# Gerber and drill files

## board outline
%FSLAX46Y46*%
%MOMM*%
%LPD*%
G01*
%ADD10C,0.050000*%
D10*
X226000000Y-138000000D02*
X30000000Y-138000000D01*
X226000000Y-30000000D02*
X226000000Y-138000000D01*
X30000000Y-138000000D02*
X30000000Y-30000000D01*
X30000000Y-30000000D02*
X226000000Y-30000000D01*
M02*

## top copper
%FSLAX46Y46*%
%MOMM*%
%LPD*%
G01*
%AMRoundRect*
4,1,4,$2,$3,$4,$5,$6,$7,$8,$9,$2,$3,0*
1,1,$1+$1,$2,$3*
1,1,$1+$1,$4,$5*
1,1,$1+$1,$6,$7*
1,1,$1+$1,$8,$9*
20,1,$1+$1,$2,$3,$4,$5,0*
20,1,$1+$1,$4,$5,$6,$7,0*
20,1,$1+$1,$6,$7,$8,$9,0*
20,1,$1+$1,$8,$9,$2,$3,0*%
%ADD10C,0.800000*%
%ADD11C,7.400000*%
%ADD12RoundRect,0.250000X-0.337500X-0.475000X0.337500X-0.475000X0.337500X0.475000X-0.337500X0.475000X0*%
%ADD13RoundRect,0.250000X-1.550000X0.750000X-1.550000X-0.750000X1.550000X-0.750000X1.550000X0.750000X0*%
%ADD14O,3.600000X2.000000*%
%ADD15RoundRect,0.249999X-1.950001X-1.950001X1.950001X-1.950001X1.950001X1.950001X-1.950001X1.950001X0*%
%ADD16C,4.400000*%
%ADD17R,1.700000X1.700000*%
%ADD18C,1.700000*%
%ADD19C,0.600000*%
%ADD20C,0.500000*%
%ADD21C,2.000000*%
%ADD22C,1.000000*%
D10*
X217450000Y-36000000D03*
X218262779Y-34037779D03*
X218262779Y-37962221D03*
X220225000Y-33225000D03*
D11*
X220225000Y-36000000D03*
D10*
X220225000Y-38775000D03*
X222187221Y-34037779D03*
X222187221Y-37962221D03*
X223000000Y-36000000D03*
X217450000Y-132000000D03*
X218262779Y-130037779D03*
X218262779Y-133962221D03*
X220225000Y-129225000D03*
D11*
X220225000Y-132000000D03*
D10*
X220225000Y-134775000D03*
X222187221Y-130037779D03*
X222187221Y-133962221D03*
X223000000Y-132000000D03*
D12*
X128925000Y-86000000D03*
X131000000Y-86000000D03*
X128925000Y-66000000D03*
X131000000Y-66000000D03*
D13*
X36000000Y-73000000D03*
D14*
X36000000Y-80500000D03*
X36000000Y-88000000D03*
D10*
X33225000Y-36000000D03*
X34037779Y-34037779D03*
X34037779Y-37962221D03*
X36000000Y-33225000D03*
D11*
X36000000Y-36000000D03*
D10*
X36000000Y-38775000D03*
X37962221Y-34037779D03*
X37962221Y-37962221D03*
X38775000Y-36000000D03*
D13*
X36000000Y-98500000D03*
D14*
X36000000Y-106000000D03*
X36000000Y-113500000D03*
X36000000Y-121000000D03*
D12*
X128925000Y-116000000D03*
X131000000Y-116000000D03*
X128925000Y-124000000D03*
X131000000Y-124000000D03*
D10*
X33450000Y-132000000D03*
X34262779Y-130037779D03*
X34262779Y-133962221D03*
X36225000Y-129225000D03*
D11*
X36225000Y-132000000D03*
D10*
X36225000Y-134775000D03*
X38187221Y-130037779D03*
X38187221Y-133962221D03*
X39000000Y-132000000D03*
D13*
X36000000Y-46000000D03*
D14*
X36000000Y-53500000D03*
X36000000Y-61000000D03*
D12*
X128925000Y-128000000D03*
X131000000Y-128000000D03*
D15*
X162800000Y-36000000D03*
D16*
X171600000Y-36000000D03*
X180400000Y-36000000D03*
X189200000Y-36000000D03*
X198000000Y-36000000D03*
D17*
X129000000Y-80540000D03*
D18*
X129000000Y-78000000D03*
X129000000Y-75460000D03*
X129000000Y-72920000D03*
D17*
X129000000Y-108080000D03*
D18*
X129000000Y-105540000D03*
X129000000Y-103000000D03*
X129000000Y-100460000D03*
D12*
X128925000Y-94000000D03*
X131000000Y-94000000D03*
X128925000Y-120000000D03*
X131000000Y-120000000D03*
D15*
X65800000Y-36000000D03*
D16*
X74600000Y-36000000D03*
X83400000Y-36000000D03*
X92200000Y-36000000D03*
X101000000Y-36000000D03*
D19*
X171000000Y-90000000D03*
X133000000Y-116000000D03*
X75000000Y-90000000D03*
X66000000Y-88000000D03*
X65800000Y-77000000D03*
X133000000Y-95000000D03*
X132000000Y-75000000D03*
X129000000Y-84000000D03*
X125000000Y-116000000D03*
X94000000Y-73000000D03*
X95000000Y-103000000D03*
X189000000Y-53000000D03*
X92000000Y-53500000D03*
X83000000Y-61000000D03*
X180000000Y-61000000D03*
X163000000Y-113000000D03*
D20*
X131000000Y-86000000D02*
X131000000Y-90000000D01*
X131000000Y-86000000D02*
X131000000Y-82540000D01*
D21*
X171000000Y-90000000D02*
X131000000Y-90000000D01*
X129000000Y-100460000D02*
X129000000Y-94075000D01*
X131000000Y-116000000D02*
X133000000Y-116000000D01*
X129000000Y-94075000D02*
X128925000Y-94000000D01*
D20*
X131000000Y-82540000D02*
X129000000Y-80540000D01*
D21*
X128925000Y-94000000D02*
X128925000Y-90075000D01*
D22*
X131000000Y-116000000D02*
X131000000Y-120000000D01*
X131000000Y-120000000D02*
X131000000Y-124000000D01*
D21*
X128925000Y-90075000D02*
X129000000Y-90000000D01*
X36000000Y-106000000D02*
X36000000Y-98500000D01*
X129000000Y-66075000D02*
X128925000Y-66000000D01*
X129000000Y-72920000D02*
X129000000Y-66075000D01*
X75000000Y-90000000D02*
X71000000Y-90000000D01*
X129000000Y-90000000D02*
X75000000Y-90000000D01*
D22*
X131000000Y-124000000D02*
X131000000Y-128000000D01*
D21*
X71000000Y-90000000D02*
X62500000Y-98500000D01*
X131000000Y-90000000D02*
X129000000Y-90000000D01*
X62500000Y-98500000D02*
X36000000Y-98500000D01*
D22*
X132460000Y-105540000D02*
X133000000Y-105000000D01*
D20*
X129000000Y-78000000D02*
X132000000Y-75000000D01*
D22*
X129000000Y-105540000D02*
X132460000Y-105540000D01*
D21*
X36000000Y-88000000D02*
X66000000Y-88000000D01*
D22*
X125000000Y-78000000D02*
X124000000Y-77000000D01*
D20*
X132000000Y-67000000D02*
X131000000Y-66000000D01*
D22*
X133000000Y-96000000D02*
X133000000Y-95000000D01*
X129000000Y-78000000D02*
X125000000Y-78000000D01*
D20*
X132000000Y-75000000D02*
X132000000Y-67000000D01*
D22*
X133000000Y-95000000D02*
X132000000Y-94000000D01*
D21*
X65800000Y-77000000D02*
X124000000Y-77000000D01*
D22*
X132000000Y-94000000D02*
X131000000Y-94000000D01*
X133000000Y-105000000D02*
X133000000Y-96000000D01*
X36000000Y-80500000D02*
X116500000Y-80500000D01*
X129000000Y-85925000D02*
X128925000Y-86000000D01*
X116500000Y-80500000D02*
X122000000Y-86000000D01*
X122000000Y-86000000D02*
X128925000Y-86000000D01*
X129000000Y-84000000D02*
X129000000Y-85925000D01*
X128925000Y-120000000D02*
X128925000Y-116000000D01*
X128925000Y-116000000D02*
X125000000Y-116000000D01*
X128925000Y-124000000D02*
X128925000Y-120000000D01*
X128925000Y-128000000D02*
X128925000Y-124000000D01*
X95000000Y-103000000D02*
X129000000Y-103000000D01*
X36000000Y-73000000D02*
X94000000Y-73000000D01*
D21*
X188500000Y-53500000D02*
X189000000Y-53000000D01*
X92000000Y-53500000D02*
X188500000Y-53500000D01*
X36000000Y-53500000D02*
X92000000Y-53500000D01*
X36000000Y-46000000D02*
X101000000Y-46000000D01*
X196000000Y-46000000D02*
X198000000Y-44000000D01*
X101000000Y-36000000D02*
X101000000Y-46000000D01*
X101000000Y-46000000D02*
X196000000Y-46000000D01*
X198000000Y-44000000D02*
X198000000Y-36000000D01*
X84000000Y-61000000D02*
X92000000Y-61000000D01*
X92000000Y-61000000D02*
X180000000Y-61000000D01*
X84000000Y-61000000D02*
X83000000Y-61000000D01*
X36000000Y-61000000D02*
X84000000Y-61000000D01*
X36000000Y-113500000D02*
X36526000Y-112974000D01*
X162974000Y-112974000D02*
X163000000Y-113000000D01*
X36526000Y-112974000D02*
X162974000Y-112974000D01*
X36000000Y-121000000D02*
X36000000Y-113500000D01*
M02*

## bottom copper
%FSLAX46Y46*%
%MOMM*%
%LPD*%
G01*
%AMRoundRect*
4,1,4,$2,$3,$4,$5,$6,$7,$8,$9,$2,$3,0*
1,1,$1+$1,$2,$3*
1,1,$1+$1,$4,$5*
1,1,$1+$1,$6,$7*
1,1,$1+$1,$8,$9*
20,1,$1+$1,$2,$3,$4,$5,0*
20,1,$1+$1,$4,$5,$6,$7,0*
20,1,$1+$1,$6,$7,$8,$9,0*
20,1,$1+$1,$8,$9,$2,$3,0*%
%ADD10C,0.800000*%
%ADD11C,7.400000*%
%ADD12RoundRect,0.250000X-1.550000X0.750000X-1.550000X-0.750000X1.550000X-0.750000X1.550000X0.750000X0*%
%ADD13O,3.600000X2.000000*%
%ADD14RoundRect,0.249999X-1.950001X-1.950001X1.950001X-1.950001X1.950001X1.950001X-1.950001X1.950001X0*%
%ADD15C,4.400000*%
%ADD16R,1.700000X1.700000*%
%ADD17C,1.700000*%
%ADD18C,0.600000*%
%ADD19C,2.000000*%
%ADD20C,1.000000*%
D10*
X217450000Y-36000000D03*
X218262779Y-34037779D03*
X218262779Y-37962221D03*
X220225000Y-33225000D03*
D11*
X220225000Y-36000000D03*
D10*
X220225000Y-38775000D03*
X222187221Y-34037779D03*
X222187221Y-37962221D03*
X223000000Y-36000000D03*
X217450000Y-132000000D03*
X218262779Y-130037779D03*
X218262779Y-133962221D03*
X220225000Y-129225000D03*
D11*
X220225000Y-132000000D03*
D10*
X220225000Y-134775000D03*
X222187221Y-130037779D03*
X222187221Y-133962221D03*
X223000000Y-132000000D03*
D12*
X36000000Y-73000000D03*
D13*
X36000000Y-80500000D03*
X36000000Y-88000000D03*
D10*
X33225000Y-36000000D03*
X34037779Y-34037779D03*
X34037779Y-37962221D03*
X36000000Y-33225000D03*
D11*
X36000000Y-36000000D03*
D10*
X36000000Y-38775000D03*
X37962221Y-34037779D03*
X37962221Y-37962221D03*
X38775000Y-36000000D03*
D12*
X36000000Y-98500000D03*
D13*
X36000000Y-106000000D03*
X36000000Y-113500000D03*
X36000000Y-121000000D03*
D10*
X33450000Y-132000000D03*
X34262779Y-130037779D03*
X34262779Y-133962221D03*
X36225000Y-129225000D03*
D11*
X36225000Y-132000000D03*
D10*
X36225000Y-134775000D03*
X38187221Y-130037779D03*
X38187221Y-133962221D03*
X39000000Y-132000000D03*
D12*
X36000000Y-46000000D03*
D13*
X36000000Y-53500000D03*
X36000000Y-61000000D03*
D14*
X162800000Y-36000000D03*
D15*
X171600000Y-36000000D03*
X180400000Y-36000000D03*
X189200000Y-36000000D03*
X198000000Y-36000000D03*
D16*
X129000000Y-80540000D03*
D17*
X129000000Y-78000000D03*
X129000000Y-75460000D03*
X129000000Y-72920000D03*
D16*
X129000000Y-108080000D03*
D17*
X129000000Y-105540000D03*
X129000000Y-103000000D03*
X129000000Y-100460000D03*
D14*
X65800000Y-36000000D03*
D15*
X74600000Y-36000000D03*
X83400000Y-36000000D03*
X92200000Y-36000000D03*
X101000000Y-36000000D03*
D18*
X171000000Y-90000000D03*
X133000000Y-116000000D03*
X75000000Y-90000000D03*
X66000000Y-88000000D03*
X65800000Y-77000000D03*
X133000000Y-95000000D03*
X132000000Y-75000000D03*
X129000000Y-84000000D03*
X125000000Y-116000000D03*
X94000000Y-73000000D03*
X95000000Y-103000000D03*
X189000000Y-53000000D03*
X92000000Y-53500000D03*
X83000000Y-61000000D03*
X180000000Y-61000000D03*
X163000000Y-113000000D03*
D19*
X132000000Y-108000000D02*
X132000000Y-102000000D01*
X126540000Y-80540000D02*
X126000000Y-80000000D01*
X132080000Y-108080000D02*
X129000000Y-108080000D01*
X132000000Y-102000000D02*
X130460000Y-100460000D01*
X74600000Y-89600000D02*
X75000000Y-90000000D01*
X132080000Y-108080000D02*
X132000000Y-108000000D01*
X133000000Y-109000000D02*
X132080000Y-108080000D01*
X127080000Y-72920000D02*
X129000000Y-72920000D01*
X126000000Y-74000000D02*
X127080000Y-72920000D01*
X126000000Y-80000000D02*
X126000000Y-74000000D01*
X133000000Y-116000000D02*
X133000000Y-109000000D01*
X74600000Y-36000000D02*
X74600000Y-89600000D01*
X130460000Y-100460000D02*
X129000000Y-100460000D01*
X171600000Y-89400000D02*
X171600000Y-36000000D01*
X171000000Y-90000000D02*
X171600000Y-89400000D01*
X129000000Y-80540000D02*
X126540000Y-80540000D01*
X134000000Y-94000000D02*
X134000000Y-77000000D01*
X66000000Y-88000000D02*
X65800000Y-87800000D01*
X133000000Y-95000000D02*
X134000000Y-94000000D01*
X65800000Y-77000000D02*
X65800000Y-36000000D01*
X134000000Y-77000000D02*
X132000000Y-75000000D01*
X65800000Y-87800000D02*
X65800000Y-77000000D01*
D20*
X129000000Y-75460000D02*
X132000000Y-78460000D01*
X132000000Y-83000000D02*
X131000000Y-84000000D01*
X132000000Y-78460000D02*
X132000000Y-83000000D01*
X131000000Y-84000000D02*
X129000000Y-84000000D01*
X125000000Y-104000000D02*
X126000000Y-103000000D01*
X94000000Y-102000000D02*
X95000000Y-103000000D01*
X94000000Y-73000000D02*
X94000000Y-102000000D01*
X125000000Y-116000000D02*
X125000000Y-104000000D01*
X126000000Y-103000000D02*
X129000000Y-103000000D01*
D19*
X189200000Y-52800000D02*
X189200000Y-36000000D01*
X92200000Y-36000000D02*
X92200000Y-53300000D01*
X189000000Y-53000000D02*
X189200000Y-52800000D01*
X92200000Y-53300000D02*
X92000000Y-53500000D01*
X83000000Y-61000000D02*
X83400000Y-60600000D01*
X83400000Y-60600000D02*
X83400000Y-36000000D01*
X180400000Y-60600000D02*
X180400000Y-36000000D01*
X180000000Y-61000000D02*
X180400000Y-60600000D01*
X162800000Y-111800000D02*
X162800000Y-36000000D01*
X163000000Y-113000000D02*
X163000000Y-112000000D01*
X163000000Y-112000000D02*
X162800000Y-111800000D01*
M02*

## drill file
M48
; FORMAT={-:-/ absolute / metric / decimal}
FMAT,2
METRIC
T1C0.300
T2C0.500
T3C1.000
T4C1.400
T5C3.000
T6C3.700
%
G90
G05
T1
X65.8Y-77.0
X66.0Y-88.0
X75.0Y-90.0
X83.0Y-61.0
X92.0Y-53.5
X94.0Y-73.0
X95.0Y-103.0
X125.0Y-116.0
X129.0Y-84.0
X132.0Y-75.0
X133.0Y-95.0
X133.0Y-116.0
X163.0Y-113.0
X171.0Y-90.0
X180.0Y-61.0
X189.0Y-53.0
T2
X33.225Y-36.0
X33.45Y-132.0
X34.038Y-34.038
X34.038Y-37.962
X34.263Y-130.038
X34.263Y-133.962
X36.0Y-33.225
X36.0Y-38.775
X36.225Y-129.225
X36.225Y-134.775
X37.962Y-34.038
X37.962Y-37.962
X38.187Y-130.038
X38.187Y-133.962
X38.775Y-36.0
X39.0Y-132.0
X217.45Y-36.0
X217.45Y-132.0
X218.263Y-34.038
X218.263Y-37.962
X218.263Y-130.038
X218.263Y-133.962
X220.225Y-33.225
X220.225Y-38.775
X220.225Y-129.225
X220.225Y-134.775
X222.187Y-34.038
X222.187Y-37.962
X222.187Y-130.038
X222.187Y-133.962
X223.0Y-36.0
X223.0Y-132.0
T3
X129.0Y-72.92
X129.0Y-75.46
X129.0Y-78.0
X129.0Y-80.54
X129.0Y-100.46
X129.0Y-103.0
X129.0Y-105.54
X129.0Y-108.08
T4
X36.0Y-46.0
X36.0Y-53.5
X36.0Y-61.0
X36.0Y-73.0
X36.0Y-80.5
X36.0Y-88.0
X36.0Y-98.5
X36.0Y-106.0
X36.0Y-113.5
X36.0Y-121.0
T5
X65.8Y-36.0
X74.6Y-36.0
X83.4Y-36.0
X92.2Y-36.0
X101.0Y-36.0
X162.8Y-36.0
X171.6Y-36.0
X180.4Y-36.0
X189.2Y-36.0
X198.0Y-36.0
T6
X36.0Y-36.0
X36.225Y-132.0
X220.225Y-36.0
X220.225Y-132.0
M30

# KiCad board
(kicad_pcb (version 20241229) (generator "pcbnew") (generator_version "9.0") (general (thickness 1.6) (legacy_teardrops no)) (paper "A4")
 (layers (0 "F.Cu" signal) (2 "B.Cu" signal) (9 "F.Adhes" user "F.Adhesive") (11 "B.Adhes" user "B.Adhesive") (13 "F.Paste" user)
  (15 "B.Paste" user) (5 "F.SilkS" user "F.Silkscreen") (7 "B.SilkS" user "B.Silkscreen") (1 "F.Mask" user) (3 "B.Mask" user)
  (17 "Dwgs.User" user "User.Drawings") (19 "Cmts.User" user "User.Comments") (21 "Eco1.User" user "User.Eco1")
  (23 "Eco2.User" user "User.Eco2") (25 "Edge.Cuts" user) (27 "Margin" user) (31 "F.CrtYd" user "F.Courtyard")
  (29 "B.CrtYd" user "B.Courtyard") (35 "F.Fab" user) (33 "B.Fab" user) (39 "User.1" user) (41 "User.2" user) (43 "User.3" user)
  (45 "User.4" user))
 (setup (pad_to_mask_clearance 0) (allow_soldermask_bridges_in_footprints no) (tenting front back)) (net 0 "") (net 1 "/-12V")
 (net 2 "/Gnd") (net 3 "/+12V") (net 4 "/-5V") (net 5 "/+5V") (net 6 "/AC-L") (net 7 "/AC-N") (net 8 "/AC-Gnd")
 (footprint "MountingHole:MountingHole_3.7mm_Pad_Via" (layer "F.Cu") (at 220.225 36)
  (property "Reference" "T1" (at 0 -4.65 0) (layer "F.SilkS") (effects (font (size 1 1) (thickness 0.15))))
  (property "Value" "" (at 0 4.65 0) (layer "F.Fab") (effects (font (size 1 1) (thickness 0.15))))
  (pad "1" thru_hole circle (at -2.775 0) (size 0.8 0.8) (drill 0.5) (layers "*.Cu" "*.Mask") (remove_unused_layers no) (zone_connect 2))
  (pad "1" thru_hole circle (at -1.962221 -1.962221) (size 0.8 0.8) (drill 0.5) (layers "*.Cu" "*.Mask") (remove_unused_layers no)
   (zone_connect 2))
  (pad "1" thru_hole circle (at -1.962221 1.962221) (size 0.8 0.8) (drill 0.5) (layers "*.Cu" "*.Mask") (remove_unused_layers no)
   (zone_connect 2))
  (pad "1" thru_hole circle (at 0 -2.775) (size 0.8 0.8) (drill 0.5) (layers "*.Cu" "*.Mask") (remove_unused_layers no) (zone_connect 2))
  (pad "1" thru_hole circle (at 0 0) (size 7.4 7.4) (drill 3.7) (layers "*.Cu" "*.Mask") (remove_unused_layers no) (zone_connect 2))
  (pad "1" thru_hole circle (at 0 2.775) (size 0.8 0.8) (drill 0.5) (layers "*.Cu" "*.Mask") (remove_unused_layers no) (zone_connect 2))
  (pad "1" thru_hole circle (at 1.962221 -1.962221) (size 0.8 0.8) (drill 0.5) (layers "*.Cu" "*.Mask") (remove_unused_layers no)
   (zone_connect 2))
  (pad "1" thru_hole circle (at 1.962221 1.962221) (size 0.8 0.8) (drill 0.5) (layers "*.Cu" "*.Mask") (remove_unused_layers no)
   (zone_connect 2))
  (pad "1" thru_hole circle (at 2.775 0) (size 0.8 0.8) (drill 0.5) (layers "*.Cu" "*.Mask") (remove_unused_layers no) (zone_connect 2)))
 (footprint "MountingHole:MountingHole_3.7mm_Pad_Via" (layer "F.Cu") (at 220.225 132)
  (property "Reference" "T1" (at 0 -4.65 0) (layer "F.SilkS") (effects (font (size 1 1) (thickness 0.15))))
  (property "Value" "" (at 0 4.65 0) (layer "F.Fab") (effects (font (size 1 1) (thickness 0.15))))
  (pad "1" thru_hole circle (at -2.775 0) (size 0.8 0.8) (drill 0.5) (layers "*.Cu" "*.Mask") (remove_unused_layers no) (zone_connect 2))
  (pad "1" thru_hole circle (at -1.962221 -1.962221) (size 0.8 0.8) (drill 0.5) (layers "*.Cu" "*.Mask") (remove_unused_layers no)
   (zone_connect 2))
  (pad "1" thru_hole circle (at -1.962221 1.962221) (size 0.8 0.8) (drill 0.5) (layers "*.Cu" "*.Mask") (remove_unused_layers no)
   (zone_connect 2))
  (pad "1" thru_hole circle (at 0 -2.775) (size 0.8 0.8) (drill 0.5) (layers "*.Cu" "*.Mask") (remove_unused_layers no) (zone_connect 2))
  (pad "1" thru_hole circle (at 0 0) (size 7.4 7.4) (drill 3.7) (layers "*.Cu" "*.Mask") (remove_unused_layers no) (zone_connect 2))
  (pad "1" thru_hole circle (at 0 2.775) (size 0.8 0.8) (drill 0.5) (layers "*.Cu" "*.Mask") (remove_unused_layers no) (zone_connect 2))
  (pad "1" thru_hole circle (at 1.962221 -1.962221) (size 0.8 0.8) (drill 0.5) (layers "*.Cu" "*.Mask") (remove_unused_layers no)
   (zone_connect 2))
  (pad "1" thru_hole circle (at 1.962221 1.962221) (size 0.8 0.8) (drill 0.5) (layers "*.Cu" "*.Mask") (remove_unused_layers no)
   (zone_connect 2))
  (pad "1" thru_hole circle (at 2.775 0) (size 0.8 0.8) (drill 0.5) (layers "*.Cu" "*.Mask") (remove_unused_layers no) (zone_connect 2)))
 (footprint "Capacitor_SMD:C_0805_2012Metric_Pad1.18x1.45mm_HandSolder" (layer "F.Cu") (at 129.9625 86)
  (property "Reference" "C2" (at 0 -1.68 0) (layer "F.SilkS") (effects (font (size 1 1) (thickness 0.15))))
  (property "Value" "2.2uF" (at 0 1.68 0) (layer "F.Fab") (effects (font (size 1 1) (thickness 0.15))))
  (pad "1" smd roundrect (at -1.0375 0) (size 1.175 1.45) (layers "F.Cu" "F.Mask" "F.Paste") (roundrect_rratio 0.212766) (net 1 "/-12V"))
  (pad "2" smd roundrect (at 1.0375 0) (size 1.175 1.45) (layers "F.Cu" "F.Mask" "F.Paste") (roundrect_rratio 0.212766) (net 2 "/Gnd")))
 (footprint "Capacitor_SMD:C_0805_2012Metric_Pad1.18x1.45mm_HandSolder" (layer "F.Cu") (at 129.9625 66)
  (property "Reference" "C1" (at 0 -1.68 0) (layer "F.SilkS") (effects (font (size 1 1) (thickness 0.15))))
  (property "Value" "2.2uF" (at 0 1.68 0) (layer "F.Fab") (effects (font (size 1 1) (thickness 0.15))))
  (pad "1" smd roundrect (at -1.0375 0) (size 1.175 1.45) (layers "F.Cu" "F.Mask" "F.Paste") (roundrect_rratio 0.212766) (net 2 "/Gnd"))
  (pad "2" smd roundrect (at 1.0375 0) (size 1.175 1.45) (layers "F.Cu" "F.Mask" "F.Paste") (roundrect_rratio 0.212766) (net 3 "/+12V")))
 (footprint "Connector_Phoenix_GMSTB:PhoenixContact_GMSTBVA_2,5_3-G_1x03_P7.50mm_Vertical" (layer "F.Cu") (at 36 73 -90)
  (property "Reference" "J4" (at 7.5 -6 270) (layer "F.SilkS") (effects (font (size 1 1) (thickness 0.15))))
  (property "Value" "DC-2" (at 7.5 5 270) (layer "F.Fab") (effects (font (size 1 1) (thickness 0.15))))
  (pad "1" thru_hole roundrect (at 0 0 270) (size 2 3.6) (drill 1.4) (layers "*.Cu" "*.Mask") (remove_unused_layers no)
   (roundrect_rratio 0.125) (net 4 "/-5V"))
  (pad "2" thru_hole oval (at 7.5 0 270) (size 2 3.6) (drill 1.4) (layers "*.Cu" "*.Mask") (remove_unused_layers no) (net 1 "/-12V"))
  (pad "3" thru_hole oval (at 15 0 270) (size 2 3.6) (drill 1.4) (layers "*.Cu" "*.Mask") (remove_unused_layers no) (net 3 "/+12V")))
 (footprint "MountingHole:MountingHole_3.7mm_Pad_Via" (layer "F.Cu") (at 36 36)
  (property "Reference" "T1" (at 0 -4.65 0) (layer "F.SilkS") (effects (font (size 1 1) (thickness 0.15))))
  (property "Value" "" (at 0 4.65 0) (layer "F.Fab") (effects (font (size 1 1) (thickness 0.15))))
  (pad "1" thru_hole circle (at -2.775 0) (size 0.8 0.8) (drill 0.5) (layers "*.Cu" "*.Mask") (remove_unused_layers no) (zone_connect 2))
  (pad "1" thru_hole circle (at -1.962221 -1.962221) (size 0.8 0.8) (drill 0.5) (layers "*.Cu" "*.Mask") (remove_unused_layers no)
   (zone_connect 2))
  (pad "1" thru_hole circle (at -1.962221 1.962221) (size 0.8 0.8) (drill 0.5) (layers "*.Cu" "*.Mask") (remove_unused_layers no)
   (zone_connect 2))
  (pad "1" thru_hole circle (at 0 -2.775) (size 0.8 0.8) (drill 0.5) (layers "*.Cu" "*.Mask") (remove_unused_layers no) (zone_connect 2))
  (pad "1" thru_hole circle (at 0 0) (size 7.4 7.4) (drill 3.7) (layers "*.Cu" "*.Mask") (remove_unused_layers no) (zone_connect 2))
  (pad "1" thru_hole circle (at 0 2.775) (size 0.8 0.8) (drill 0.5) (layers "*.Cu" "*.Mask") (remove_unused_layers no) (zone_connect 2))
  (pad "1" thru_hole circle (at 1.962221 -1.962221) (size 0.8 0.8) (drill 0.5) (layers "*.Cu" "*.Mask") (remove_unused_layers no)
   (zone_connect 2))
  (pad "1" thru_hole circle (at 1.962221 1.962221) (size 0.8 0.8) (drill 0.5) (layers "*.Cu" "*.Mask") (remove_unused_layers no)
   (zone_connect 2))
  (pad "1" thru_hole circle (at 2.775 0) (size 0.8 0.8) (drill 0.5) (layers "*.Cu" "*.Mask") (remove_unused_layers no) (zone_connect 2)))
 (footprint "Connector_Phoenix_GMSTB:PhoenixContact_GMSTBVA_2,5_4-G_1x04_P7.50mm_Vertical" (layer "F.Cu") (at 36 98.5 -90)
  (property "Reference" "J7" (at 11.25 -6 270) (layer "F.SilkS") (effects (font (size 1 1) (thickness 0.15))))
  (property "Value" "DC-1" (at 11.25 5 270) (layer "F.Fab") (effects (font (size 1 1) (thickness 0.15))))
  (pad "1" thru_hole roundrect (at 0 0 270) (size 2 3.6) (drill 1.4) (layers "*.Cu" "*.Mask") (remove_unused_layers no)
   (roundrect_rratio 0.125) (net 2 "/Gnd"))
  (pad "2" thru_hole oval (at 7.5 0 270) (size 2 3.6) (drill 1.4) (layers "*.Cu" "*.Mask") (remove_unused_layers no) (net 2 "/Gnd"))
  (pad "3" thru_hole oval (at 15 0 270) (size 2 3.6) (drill 1.4) (layers "*.Cu" "*.Mask") (remove_unused_layers no) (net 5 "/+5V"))
  (pad "4" thru_hole oval (at 22.5 0 270) (size 2 3.6) (drill 1.4) (layers "*.Cu" "*.Mask") (remove_unused_layers no) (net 5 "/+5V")))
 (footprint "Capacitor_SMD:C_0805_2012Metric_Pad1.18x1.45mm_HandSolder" (layer "F.Cu") (at 129.9625 116)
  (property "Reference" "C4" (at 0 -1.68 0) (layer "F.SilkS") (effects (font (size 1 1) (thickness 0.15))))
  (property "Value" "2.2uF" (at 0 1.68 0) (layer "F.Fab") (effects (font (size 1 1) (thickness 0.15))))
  (pad "1" smd roundrect (at -1.0375 0) (size 1.175 1.45) (layers "F.Cu" "F.Mask" "F.Paste") (roundrect_rratio 0.212766) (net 4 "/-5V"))
  (pad "2" smd roundrect (at 1.0375 0) (size 1.175 1.45) (layers "F.Cu" "F.Mask" "F.Paste") (roundrect_rratio 0.212766) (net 2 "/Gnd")))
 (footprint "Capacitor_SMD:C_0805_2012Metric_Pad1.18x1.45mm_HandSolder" (layer "F.Cu") (at 129.9625 124)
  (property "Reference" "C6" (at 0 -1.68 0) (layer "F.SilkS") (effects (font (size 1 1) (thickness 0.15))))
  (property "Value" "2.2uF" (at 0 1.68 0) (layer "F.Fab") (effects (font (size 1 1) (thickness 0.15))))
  (pad "1" smd roundrect (at -1.0375 0) (size 1.175 1.45) (layers "F.Cu" "F.Mask" "F.Paste") (roundrect_rratio 0.212766) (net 4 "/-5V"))
  (pad "2" smd roundrect (at 1.0375 0) (size 1.175 1.45) (layers "F.Cu" "F.Mask" "F.Paste") (roundrect_rratio 0.212766) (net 2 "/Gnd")))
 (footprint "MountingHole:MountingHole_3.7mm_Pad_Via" (layer "F.Cu") (at 36.225 132)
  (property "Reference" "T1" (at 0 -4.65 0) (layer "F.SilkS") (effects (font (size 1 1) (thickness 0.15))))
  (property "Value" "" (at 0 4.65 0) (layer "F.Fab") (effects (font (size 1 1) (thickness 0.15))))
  (pad "1" thru_hole circle (at -2.775 0) (size 0.8 0.8) (drill 0.5) (layers "*.Cu" "*.Mask") (remove_unused_layers no) (zone_connect 2))
  (pad "1" thru_hole circle (at -1.962221 -1.962221) (size 0.8 0.8) (drill 0.5) (layers "*.Cu" "*.Mask") (remove_unused_layers no)
   (zone_connect 2))
  (pad "1" thru_hole circle (at -1.962221 1.962221) (size 0.8 0.8) (drill 0.5) (layers "*.Cu" "*.Mask") (remove_unused_layers no)
   (zone_connect 2))
  (pad "1" thru_hole circle (at 0 -2.775) (size 0.8 0.8) (drill 0.5) (layers "*.Cu" "*.Mask") (remove_unused_layers no) (zone_connect 2))
  (pad "1" thru_hole circle (at 0 0) (size 7.4 7.4) (drill 3.7) (layers "*.Cu" "*.Mask") (remove_unused_layers no) (zone_connect 2))
  (pad "1" thru_hole circle (at 0 2.775) (size 0.8 0.8) (drill 0.5) (layers "*.Cu" "*.Mask") (remove_unused_layers no) (zone_connect 2))
  (pad "1" thru_hole circle (at 1.962221 -1.962221) (size 0.8 0.8) (drill 0.5) (layers "*.Cu" "*.Mask") (remove_unused_layers no)
   (zone_connect 2))
  (pad "1" thru_hole circle (at 1.962221 1.962221) (size 0.8 0.8) (drill 0.5) (layers "*.Cu" "*.Mask") (remove_unused_layers no)
   (zone_connect 2))
  (pad "1" thru_hole circle (at 2.775 0) (size 0.8 0.8) (drill 0.5) (layers "*.Cu" "*.Mask") (remove_unused_layers no) (zone_connect 2)))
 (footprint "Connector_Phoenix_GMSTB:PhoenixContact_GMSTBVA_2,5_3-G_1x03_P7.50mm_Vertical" (layer "F.Cu") (at 36 46 -90)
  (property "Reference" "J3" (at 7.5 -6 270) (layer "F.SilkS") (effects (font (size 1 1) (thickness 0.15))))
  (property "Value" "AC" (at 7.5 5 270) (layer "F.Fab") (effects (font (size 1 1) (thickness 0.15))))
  (pad "1" thru_hole roundrect (at 0 0 270) (size 2 3.6) (drill 1.4) (layers "*.Cu" "*.Mask") (remove_unused_layers no)
   (roundrect_rratio 0.125) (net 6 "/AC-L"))
  (pad "2" thru_hole oval (at 7.5 0 270) (size 2 3.6) (drill 1.4) (layers "*.Cu" "*.Mask") (remove_unused_layers no) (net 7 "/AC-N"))
  (pad "3" thru_hole oval (at 15 0 270) (size 2 3.6) (drill 1.4) (layers "*.Cu" "*.Mask") (remove_unused_layers no) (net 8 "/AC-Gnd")))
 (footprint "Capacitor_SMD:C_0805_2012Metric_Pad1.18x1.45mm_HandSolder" (layer "F.Cu") (at 129.9625 128)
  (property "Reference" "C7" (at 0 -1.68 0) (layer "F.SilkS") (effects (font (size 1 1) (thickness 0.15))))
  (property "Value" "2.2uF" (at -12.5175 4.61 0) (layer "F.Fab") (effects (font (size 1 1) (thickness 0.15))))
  (pad "1" smd roundrect (at -1.0375 0) (size 1.175 1.45) (layers "F.Cu" "F.Mask" "F.Paste") (roundrect_rratio 0.212766) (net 4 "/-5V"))
  (pad "2" smd roundrect (at 1.0375 0) (size 1.175 1.45) (layers "F.Cu" "F.Mask" "F.Paste") (roundrect_rratio 0.212766) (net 2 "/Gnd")))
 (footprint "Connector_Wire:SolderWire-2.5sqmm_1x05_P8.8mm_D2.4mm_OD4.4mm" (layer "F.Cu") (at 162.8 36)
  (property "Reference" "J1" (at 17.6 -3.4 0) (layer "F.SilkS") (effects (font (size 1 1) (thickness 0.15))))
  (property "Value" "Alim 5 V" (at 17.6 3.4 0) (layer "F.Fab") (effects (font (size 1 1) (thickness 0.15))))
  (pad "1" thru_hole roundrect (at 0 0) (size 4.4 4.4) (drill 3) (layers "*.Cu" "*.Mask") (remove_unused_layers no)
   (roundrect_rratio 0.056818) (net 5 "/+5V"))
  (pad "2" thru_hole circle (at 8.8 0) (size 4.4 4.4) (drill 3) (layers "*.Cu" "*.Mask") (remove_unused_layers no) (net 2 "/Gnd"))
  (pad "3" thru_hole circle (at 17.6 0) (size 4.4 4.4) (drill 3) (layers "*.Cu" "*.Mask") (remove_unused_layers no) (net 8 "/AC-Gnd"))
  (pad "4" thru_hole circle (at 26.4 0) (size 4.4 4.4) (drill 3) (layers "*.Cu" "*.Mask") (remove_unused_layers no) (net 7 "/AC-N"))
  (pad "5" thru_hole circle (at 35.2 0) (size 4.4 4.4) (drill 3) (layers "*.Cu" "*.Mask") (remove_unused_layers no) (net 6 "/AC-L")))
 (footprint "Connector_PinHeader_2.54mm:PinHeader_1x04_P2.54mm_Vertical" (layer "F.Cu") (at 129 80.54 180)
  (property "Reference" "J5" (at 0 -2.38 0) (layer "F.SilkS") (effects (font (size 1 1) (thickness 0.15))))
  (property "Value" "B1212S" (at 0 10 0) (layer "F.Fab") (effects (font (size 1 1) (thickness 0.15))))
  (pad "1" thru_hole rect (at 0 0 180) (size 1.7 1.7) (drill 1) (layers "*.Cu" "*.Mask") (remove_unused_layers no) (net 2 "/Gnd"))
  (pad "2" thru_hole circle (at 0 2.54 180) (size 1.7 1.7) (drill 1) (layers "*.Cu" "*.Mask") (remove_unused_layers no) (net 3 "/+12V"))
  (pad "3" thru_hole circle (at 0 5.08 180) (size 1.7 1.7) (drill 1) (layers "*.Cu" "*.Mask") (remove_unused_layers no) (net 1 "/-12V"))
  (pad "4" thru_hole circle (at 0 7.62 180) (size 1.7 1.7) (drill 1) (layers "*.Cu" "*.Mask") (remove_unused_layers no) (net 2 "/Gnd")))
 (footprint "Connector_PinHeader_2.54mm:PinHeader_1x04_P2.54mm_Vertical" (layer "F.Cu") (at 129 108.08 180)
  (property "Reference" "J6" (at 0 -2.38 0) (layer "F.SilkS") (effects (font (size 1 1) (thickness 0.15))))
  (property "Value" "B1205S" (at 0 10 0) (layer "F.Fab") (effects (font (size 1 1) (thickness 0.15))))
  (pad "1" thru_hole rect (at 0 0 180) (size 1.7 1.7) (drill 1) (layers "*.Cu" "*.Mask") (remove_unused_layers no) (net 2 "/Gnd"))
  (pad "2" thru_hole circle (at 0 2.54 180) (size 1.7 1.7) (drill 1) (layers "*.Cu" "*.Mask") (remove_unused_layers no) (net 3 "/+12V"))
  (pad "3" thru_hole circle (at 0 5.08 180) (size 1.7 1.7) (drill 1) (layers "*.Cu" "*.Mask") (remove_unused_layers no) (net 4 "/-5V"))
  (pad "4" thru_hole circle (at 0 7.62 180) (size 1.7 1.7) (drill 1) (layers "*.Cu" "*.Mask") (remove_unused_layers no) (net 2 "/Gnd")))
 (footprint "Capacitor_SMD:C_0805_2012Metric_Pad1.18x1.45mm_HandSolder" (layer "F.Cu") (at 129.9625 94)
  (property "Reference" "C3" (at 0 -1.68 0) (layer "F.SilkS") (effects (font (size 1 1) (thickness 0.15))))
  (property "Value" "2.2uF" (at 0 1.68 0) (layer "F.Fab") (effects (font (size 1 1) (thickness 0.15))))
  (pad "1" smd roundrect (at -1.0375 0) (size 1.175 1.45) (layers "F.Cu" "F.Mask" "F.Paste") (roundrect_rratio 0.212766) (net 2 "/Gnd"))
  (pad "2" smd roundrect (at 1.0375 0) (size 1.175 1.45) (layers "F.Cu" "F.Mask" "F.Paste") (roundrect_rratio 0.212766) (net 3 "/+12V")))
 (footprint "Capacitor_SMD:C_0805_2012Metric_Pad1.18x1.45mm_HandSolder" (layer "F.Cu") (at 129.9625 120)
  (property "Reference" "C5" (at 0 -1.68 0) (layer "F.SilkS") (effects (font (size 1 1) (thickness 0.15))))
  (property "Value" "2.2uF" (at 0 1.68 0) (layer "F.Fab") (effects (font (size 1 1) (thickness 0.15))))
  (pad "1" smd roundrect (at -1.0375 0) (size 1.175 1.45) (layers "F.Cu" "F.Mask" "F.Paste") (roundrect_rratio 0.212766) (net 4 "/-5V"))
  (pad "2" smd roundrect (at 1.0375 0) (size 1.175 1.45) (layers "F.Cu" "F.Mask" "F.Paste") (roundrect_rratio 0.212766) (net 2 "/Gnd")))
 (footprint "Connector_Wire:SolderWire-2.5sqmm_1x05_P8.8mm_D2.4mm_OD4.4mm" (layer "F.Cu") (at 65.8 36)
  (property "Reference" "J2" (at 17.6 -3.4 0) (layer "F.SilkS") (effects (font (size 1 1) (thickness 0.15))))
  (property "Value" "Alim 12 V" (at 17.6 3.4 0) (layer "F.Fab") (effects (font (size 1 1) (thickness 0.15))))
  (pad "1" thru_hole roundrect (at 0 0) (size 4.4 4.4) (drill 3) (layers "*.Cu" "*.Mask") (remove_unused_layers no)
   (roundrect_rratio 0.056818) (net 3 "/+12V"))
  (pad "2" thru_hole circle (at 8.8 0) (size 4.4 4.4) (drill 3) (layers "*.Cu" "*.Mask") (remove_unused_layers no) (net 2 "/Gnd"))
  (pad "3" thru_hole circle (at 17.6 0) (size 4.4 4.4) (drill 3) (layers "*.Cu" "*.Mask") (remove_unused_layers no) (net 8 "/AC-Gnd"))
  (pad "4" thru_hole circle (at 26.4 0) (size 4.4 4.4) (drill 3) (layers "*.Cu" "*.Mask") (remove_unused_layers no) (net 7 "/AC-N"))
  (pad "5" thru_hole circle (at 35.2 0) (size 4.4 4.4) (drill 3) (layers "*.Cu" "*.Mask") (remove_unused_layers no) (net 6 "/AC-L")))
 (gr_line (start 226 138) (end 30 138) (stroke (width 0.05) (type default)) (layer "Edge.Cuts"))
 (gr_line (start 226 30) (end 226 138) (stroke (width 0.05) (type default)) (layer "Edge.Cuts"))
 (gr_line (start 30 138) (end 30 30) (stroke (width 0.05) (type default)) (layer "Edge.Cuts"))
 (gr_line (start 30 30) (end 226 30) (stroke (width 0.05) (type default)) (layer "Edge.Cuts"))
 (segment (start 131 86) (end 131 90) (width 0.5) (layer "F.Cu") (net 2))
 (segment (start 131 86) (end 131 82.54) (width 0.5) (layer "F.Cu") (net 2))
 (segment (start 171 90) (end 131 90) (width 2) (layer "F.Cu") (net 2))
 (segment (start 129 100.46) (end 129 94.075) (width 2) (layer "F.Cu") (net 2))
 (segment (start 131 116) (end 133 116) (width 2) (layer "F.Cu") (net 2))
 (segment (start 129 94.075) (end 128.925 94) (width 2) (layer "F.Cu") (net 2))
 (segment (start 131 82.54) (end 129 80.54) (width 0.5) (layer "F.Cu") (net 2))
 (segment (start 128.925 94) (end 128.925 90.075) (width 2) (layer "F.Cu") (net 2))
 (segment (start 131 116) (end 131 120) (width 1) (layer "F.Cu") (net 2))
 (segment (start 131 120) (end 131 124) (width 1) (layer "F.Cu") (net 2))
 (segment (start 128.925 90.075) (end 129 90) (width 2) (layer "F.Cu") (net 2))
 (segment (start 36 106) (end 36 98.5) (width 2) (layer "F.Cu") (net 2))
 (segment (start 129 66.075) (end 128.925 66) (width 2) (layer "F.Cu") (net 2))
 (segment (start 129 72.92) (end 129 66.075) (width 2) (layer "F.Cu") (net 2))
 (segment (start 75 90) (end 71 90) (width 2) (layer "F.Cu") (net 2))
 (segment (start 129 90) (end 75 90) (width 2) (layer "F.Cu") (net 2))
 (segment (start 131 124) (end 131 128) (width 1) (layer "F.Cu") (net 2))
 (segment (start 71 90) (end 62.5 98.5) (width 2) (layer "F.Cu") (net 2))
 (segment (start 131 90) (end 129 90) (width 2) (layer "F.Cu") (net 2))
 (segment (start 62.5 98.5) (end 36 98.5) (width 2) (layer "F.Cu") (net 2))
 (via (at 171 90) (size 0.6) (drill 0.3) (layers "F.Cu" "B.Cu") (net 2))
 (via (at 133 116) (size 0.6) (drill 0.3) (layers "F.Cu" "B.Cu") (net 2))
 (via (at 75 90) (size 0.6) (drill 0.3) (layers "F.Cu" "B.Cu") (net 2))
 (segment (start 132 108) (end 132 102) (width 2) (layer "B.Cu") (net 2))
 (segment (start 126.54 80.54) (end 126 80) (width 2) (layer "B.Cu") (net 2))
 (segment (start 132.08 108.08) (end 129 108.08) (width 2) (layer "B.Cu") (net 2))
 (segment (start 132 102) (end 130.46 100.46) (width 2) (layer "B.Cu") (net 2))
 (segment (start 74.6 89.6) (end 75 90) (width 2) (layer "B.Cu") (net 2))
 (segment (start 132.08 108.08) (end 132 108) (width 2) (layer "B.Cu") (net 2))
 (segment (start 133 109) (end 132.08 108.08) (width 2) (layer "B.Cu") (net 2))
 (segment (start 127.08 72.92) (end 129 72.92) (width 2) (layer "B.Cu") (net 2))
 (segment (start 126 74) (end 127.08 72.92) (width 2) (layer "B.Cu") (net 2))
 (segment (start 126 80) (end 126 74) (width 2) (layer "B.Cu") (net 2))
 (segment (start 133 116) (end 133 109) (width 2) (layer "B.Cu") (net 2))
 (segment (start 74.6 36) (end 74.6 89.6) (width 2) (layer "B.Cu") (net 2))
 (segment (start 130.46 100.46) (end 129 100.46) (width 2) (layer "B.Cu") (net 2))
 (segment (start 171.6 89.4) (end 171.6 36) (width 2) (layer "B.Cu") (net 2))
 (segment (start 171 90) (end 171.6 89.4) (width 2) (layer "B.Cu") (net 2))
 (segment (start 129 80.54) (end 126.54 80.54) (width 2) (layer "B.Cu") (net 2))
 (segment (start 132.46 105.54) (end 133 105) (width 1) (layer "F.Cu") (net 3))
 (segment (start 129 78) (end 132 75) (width 0.5) (layer "F.Cu") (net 3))
 (segment (start 129 105.54) (end 132.46 105.54) (width 1) (layer "F.Cu") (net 3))
 (segment (start 36 88) (end 66 88) (width 2) (layer "F.Cu") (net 3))
 (segment (start 125 78) (end 124 77) (width 1) (layer "F.Cu") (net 3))
 (segment (start 132 67) (end 131 66) (width 0.5) (layer "F.Cu") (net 3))
 (segment (start 133 96) (end 133 95) (width 1) (layer "F.Cu") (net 3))
 (segment (start 129 78) (end 125 78) (width 1) (layer "F.Cu") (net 3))
 (segment (start 132 75) (end 132 67) (width 0.5) (layer "F.Cu") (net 3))
 (segment (start 133 95) (end 132 94) (width 1) (layer "F.Cu") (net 3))
 (segment (start 65.8 77) (end 124 77) (width 2) (layer "F.Cu") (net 3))
 (segment (start 132 94) (end 131 94) (width 1) (layer "F.Cu") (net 3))
 (segment (start 133 105) (end 133 96) (width 1) (layer "F.Cu") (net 3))
 (via (at 66 88) (size 0.6) (drill 0.3) (layers "F.Cu" "B.Cu") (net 3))
 (via (at 65.8 77) (size 0.6) (drill 0.3) (layers "F.Cu" "B.Cu") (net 3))
 (via (at 133 95) (size 0.6) (drill 0.3) (layers "F.Cu" "B.Cu") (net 3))
 (via (at 132 75) (size 0.6) (drill 0.3) (layers "F.Cu" "B.Cu") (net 3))
 (segment (start 134 94) (end 134 77) (width 2) (layer "B.Cu") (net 3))
 (segment (start 66 88) (end 65.8 87.8) (width 2) (layer "B.Cu") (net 3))
 (segment (start 133 95) (end 134 94) (width 2) (layer "B.Cu") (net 3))
 (segment (start 65.8 77) (end 65.8 36) (width 2) (layer "B.Cu") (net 3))
 (segment (start 134 77) (end 132 75) (width 2) (layer "B.Cu") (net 3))
 (segment (start 65.8 87.8) (end 65.8 77) (width 2) (layer "B.Cu") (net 3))
 (segment (start 36 80.5) (end 116.5 80.5) (width 1) (layer "F.Cu") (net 1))
 (segment (start 129 85.925) (end 128.925 86) (width 1) (layer "F.Cu") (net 1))
 (segment (start 116.5 80.5) (end 122 86) (width 1) (layer "F.Cu") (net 1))
 (segment (start 122 86) (end 128.925 86) (width 1) (layer "F.Cu") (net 1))
 (segment (start 129 84) (end 129 85.925) (width 1) (layer "F.Cu") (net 1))
 (via (at 129 84) (size 0.6) (drill 0.3) (layers "F.Cu" "B.Cu") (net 1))
 (segment (start 129 75.46) (end 132 78.46) (width 1) (layer "B.Cu") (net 1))
 (segment (start 132 83) (end 131 84) (width 1) (layer "B.Cu") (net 1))
 (segment (start 132 78.46) (end 132 83) (width 1) (layer "B.Cu") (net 1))
 (segment (start 131 84) (end 129 84) (width 1) (layer "B.Cu") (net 1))
 (segment (start 128.925 120) (end 128.925 116) (width 1) (layer "F.Cu") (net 4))
 (segment (start 128.925 116) (end 125 116) (width 1) (layer "F.Cu") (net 4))
 (segment (start 128.925 124) (end 128.925 120) (width 1) (layer "F.Cu") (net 4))
 (segment (start 128.925 128) (end 128.925 124) (width 1) (layer "F.Cu") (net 4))
 (segment (start 95 103) (end 129 103) (width 1) (layer "F.Cu") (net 4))
 (segment (start 36 73) (end 94 73) (width 1) (layer "F.Cu") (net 4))
 (via (at 125 116) (size 0.6) (drill 0.3) (layers "F.Cu" "B.Cu") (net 4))
 (via (at 94 73) (size 0.6) (drill 0.3) (layers "F.Cu" "B.Cu") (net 4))
 (via (at 95 103) (size 0.6) (drill 0.3) (layers "F.Cu" "B.Cu") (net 4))
 (segment (start 125 104) (end 126 103) (width 1) (layer "B.Cu") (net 4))
 (segment (start 94 102) (end 95 103) (width 1) (layer "B.Cu") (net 4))
 (segment (start 94 73) (end 94 102) (width 1) (layer "B.Cu") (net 4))
 (segment (start 125 116) (end 125 104) (width 1) (layer "B.Cu") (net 4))
 (segment (start 126 103) (end 129 103) (width 1) (layer "B.Cu") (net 4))
 (segment (start 188.5 53.5) (end 189 53) (width 2) (layer "F.Cu") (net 7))
 (segment (start 92 53.5) (end 188.5 53.5) (width 2) (layer "F.Cu") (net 7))
 (segment (start 36 53.5) (end 92 53.5) (width 2) (layer "F.Cu") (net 7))
 (via (at 189 53) (size 0.6) (drill 0.3) (layers "F.Cu" "B.Cu") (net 7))
 (via (at 92 53.5) (size 0.6) (drill 0.3) (layers "F.Cu" "B.Cu") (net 7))
 (segment (start 189.2 52.8) (end 189.2 36) (width 2) (layer "B.Cu") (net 7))
 (segment (start 92.2 36) (end 92.2 53.3) (width 2) (layer "B.Cu") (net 7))
 (segment (start 189 53) (end 189.2 52.8) (width 2) (layer "B.Cu") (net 7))
 (segment (start 92.2 53.3) (end 92 53.5) (width 2) (layer "B.Cu") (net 7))
 (segment (start 36 46) (end 101 46) (width 2) (layer "F.Cu") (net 6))
 (segment (start 196 46) (end 198 44) (width 2) (layer "F.Cu") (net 6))
 (segment (start 101 36) (end 101 46) (width 2) (layer "F.Cu") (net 6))
 (segment (start 101 46) (end 196 46) (width 2) (layer "F.Cu") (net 6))
 (segment (start 198 44) (end 198 36) (width 2) (layer "F.Cu") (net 6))
 (segment (start 84 61) (end 92 61) (width 2) (layer "F.Cu") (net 8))
 (segment (start 92 61) (end 180 61) (width 2) (layer "F.Cu") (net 8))
 (segment (start 84 61) (end 83 61) (width 2) (layer "F.Cu") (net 8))
 (segment (start 36 61) (end 84 61) (width 2) (layer "F.Cu") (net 8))
 (via (at 83 61) (size 0.6) (drill 0.3) (layers "F.Cu" "B.Cu") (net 8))
 (via (at 180 61) (size 0.6) (drill 0.3) (layers "F.Cu" "B.Cu") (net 8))
 (segment (start 83 61) (end 83.4 60.6) (width 2) (layer "B.Cu") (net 8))
 (segment (start 83.4 60.6) (end 83.4 36) (width 2) (layer "B.Cu") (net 8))
 (segment (start 180.4 60.6) (end 180.4 36) (width 2) (layer "B.Cu") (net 8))
 (segment (start 180 61) (end 180.4 60.6) (width 2) (layer "B.Cu") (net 8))
 (segment (start 36 113.5) (end 36.526 112.974) (width 2) (layer "F.Cu") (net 5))
 (segment (start 162.974 112.974) (end 163 113) (width 2) (layer "F.Cu") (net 5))
 (segment (start 36.526 112.974) (end 162.974 112.974) (width 2) (layer "F.Cu") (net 5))
 (segment (start 36 121) (end 36 113.5) (width 2) (layer "F.Cu") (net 5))
 (via (at 163 113) (size 0.6) (drill 0.3) (layers "F.Cu" "B.Cu") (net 5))
 (segment (start 162.8 111.8) (end 162.8 36) (width 2) (layer "B.Cu") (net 5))
 (segment (start 163 113) (end 163 112) (width 2) (layer "B.Cu") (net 5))
 (segment (start 163 112) (end 162.8 111.8) (width 2) (layer "B.Cu") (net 5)))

